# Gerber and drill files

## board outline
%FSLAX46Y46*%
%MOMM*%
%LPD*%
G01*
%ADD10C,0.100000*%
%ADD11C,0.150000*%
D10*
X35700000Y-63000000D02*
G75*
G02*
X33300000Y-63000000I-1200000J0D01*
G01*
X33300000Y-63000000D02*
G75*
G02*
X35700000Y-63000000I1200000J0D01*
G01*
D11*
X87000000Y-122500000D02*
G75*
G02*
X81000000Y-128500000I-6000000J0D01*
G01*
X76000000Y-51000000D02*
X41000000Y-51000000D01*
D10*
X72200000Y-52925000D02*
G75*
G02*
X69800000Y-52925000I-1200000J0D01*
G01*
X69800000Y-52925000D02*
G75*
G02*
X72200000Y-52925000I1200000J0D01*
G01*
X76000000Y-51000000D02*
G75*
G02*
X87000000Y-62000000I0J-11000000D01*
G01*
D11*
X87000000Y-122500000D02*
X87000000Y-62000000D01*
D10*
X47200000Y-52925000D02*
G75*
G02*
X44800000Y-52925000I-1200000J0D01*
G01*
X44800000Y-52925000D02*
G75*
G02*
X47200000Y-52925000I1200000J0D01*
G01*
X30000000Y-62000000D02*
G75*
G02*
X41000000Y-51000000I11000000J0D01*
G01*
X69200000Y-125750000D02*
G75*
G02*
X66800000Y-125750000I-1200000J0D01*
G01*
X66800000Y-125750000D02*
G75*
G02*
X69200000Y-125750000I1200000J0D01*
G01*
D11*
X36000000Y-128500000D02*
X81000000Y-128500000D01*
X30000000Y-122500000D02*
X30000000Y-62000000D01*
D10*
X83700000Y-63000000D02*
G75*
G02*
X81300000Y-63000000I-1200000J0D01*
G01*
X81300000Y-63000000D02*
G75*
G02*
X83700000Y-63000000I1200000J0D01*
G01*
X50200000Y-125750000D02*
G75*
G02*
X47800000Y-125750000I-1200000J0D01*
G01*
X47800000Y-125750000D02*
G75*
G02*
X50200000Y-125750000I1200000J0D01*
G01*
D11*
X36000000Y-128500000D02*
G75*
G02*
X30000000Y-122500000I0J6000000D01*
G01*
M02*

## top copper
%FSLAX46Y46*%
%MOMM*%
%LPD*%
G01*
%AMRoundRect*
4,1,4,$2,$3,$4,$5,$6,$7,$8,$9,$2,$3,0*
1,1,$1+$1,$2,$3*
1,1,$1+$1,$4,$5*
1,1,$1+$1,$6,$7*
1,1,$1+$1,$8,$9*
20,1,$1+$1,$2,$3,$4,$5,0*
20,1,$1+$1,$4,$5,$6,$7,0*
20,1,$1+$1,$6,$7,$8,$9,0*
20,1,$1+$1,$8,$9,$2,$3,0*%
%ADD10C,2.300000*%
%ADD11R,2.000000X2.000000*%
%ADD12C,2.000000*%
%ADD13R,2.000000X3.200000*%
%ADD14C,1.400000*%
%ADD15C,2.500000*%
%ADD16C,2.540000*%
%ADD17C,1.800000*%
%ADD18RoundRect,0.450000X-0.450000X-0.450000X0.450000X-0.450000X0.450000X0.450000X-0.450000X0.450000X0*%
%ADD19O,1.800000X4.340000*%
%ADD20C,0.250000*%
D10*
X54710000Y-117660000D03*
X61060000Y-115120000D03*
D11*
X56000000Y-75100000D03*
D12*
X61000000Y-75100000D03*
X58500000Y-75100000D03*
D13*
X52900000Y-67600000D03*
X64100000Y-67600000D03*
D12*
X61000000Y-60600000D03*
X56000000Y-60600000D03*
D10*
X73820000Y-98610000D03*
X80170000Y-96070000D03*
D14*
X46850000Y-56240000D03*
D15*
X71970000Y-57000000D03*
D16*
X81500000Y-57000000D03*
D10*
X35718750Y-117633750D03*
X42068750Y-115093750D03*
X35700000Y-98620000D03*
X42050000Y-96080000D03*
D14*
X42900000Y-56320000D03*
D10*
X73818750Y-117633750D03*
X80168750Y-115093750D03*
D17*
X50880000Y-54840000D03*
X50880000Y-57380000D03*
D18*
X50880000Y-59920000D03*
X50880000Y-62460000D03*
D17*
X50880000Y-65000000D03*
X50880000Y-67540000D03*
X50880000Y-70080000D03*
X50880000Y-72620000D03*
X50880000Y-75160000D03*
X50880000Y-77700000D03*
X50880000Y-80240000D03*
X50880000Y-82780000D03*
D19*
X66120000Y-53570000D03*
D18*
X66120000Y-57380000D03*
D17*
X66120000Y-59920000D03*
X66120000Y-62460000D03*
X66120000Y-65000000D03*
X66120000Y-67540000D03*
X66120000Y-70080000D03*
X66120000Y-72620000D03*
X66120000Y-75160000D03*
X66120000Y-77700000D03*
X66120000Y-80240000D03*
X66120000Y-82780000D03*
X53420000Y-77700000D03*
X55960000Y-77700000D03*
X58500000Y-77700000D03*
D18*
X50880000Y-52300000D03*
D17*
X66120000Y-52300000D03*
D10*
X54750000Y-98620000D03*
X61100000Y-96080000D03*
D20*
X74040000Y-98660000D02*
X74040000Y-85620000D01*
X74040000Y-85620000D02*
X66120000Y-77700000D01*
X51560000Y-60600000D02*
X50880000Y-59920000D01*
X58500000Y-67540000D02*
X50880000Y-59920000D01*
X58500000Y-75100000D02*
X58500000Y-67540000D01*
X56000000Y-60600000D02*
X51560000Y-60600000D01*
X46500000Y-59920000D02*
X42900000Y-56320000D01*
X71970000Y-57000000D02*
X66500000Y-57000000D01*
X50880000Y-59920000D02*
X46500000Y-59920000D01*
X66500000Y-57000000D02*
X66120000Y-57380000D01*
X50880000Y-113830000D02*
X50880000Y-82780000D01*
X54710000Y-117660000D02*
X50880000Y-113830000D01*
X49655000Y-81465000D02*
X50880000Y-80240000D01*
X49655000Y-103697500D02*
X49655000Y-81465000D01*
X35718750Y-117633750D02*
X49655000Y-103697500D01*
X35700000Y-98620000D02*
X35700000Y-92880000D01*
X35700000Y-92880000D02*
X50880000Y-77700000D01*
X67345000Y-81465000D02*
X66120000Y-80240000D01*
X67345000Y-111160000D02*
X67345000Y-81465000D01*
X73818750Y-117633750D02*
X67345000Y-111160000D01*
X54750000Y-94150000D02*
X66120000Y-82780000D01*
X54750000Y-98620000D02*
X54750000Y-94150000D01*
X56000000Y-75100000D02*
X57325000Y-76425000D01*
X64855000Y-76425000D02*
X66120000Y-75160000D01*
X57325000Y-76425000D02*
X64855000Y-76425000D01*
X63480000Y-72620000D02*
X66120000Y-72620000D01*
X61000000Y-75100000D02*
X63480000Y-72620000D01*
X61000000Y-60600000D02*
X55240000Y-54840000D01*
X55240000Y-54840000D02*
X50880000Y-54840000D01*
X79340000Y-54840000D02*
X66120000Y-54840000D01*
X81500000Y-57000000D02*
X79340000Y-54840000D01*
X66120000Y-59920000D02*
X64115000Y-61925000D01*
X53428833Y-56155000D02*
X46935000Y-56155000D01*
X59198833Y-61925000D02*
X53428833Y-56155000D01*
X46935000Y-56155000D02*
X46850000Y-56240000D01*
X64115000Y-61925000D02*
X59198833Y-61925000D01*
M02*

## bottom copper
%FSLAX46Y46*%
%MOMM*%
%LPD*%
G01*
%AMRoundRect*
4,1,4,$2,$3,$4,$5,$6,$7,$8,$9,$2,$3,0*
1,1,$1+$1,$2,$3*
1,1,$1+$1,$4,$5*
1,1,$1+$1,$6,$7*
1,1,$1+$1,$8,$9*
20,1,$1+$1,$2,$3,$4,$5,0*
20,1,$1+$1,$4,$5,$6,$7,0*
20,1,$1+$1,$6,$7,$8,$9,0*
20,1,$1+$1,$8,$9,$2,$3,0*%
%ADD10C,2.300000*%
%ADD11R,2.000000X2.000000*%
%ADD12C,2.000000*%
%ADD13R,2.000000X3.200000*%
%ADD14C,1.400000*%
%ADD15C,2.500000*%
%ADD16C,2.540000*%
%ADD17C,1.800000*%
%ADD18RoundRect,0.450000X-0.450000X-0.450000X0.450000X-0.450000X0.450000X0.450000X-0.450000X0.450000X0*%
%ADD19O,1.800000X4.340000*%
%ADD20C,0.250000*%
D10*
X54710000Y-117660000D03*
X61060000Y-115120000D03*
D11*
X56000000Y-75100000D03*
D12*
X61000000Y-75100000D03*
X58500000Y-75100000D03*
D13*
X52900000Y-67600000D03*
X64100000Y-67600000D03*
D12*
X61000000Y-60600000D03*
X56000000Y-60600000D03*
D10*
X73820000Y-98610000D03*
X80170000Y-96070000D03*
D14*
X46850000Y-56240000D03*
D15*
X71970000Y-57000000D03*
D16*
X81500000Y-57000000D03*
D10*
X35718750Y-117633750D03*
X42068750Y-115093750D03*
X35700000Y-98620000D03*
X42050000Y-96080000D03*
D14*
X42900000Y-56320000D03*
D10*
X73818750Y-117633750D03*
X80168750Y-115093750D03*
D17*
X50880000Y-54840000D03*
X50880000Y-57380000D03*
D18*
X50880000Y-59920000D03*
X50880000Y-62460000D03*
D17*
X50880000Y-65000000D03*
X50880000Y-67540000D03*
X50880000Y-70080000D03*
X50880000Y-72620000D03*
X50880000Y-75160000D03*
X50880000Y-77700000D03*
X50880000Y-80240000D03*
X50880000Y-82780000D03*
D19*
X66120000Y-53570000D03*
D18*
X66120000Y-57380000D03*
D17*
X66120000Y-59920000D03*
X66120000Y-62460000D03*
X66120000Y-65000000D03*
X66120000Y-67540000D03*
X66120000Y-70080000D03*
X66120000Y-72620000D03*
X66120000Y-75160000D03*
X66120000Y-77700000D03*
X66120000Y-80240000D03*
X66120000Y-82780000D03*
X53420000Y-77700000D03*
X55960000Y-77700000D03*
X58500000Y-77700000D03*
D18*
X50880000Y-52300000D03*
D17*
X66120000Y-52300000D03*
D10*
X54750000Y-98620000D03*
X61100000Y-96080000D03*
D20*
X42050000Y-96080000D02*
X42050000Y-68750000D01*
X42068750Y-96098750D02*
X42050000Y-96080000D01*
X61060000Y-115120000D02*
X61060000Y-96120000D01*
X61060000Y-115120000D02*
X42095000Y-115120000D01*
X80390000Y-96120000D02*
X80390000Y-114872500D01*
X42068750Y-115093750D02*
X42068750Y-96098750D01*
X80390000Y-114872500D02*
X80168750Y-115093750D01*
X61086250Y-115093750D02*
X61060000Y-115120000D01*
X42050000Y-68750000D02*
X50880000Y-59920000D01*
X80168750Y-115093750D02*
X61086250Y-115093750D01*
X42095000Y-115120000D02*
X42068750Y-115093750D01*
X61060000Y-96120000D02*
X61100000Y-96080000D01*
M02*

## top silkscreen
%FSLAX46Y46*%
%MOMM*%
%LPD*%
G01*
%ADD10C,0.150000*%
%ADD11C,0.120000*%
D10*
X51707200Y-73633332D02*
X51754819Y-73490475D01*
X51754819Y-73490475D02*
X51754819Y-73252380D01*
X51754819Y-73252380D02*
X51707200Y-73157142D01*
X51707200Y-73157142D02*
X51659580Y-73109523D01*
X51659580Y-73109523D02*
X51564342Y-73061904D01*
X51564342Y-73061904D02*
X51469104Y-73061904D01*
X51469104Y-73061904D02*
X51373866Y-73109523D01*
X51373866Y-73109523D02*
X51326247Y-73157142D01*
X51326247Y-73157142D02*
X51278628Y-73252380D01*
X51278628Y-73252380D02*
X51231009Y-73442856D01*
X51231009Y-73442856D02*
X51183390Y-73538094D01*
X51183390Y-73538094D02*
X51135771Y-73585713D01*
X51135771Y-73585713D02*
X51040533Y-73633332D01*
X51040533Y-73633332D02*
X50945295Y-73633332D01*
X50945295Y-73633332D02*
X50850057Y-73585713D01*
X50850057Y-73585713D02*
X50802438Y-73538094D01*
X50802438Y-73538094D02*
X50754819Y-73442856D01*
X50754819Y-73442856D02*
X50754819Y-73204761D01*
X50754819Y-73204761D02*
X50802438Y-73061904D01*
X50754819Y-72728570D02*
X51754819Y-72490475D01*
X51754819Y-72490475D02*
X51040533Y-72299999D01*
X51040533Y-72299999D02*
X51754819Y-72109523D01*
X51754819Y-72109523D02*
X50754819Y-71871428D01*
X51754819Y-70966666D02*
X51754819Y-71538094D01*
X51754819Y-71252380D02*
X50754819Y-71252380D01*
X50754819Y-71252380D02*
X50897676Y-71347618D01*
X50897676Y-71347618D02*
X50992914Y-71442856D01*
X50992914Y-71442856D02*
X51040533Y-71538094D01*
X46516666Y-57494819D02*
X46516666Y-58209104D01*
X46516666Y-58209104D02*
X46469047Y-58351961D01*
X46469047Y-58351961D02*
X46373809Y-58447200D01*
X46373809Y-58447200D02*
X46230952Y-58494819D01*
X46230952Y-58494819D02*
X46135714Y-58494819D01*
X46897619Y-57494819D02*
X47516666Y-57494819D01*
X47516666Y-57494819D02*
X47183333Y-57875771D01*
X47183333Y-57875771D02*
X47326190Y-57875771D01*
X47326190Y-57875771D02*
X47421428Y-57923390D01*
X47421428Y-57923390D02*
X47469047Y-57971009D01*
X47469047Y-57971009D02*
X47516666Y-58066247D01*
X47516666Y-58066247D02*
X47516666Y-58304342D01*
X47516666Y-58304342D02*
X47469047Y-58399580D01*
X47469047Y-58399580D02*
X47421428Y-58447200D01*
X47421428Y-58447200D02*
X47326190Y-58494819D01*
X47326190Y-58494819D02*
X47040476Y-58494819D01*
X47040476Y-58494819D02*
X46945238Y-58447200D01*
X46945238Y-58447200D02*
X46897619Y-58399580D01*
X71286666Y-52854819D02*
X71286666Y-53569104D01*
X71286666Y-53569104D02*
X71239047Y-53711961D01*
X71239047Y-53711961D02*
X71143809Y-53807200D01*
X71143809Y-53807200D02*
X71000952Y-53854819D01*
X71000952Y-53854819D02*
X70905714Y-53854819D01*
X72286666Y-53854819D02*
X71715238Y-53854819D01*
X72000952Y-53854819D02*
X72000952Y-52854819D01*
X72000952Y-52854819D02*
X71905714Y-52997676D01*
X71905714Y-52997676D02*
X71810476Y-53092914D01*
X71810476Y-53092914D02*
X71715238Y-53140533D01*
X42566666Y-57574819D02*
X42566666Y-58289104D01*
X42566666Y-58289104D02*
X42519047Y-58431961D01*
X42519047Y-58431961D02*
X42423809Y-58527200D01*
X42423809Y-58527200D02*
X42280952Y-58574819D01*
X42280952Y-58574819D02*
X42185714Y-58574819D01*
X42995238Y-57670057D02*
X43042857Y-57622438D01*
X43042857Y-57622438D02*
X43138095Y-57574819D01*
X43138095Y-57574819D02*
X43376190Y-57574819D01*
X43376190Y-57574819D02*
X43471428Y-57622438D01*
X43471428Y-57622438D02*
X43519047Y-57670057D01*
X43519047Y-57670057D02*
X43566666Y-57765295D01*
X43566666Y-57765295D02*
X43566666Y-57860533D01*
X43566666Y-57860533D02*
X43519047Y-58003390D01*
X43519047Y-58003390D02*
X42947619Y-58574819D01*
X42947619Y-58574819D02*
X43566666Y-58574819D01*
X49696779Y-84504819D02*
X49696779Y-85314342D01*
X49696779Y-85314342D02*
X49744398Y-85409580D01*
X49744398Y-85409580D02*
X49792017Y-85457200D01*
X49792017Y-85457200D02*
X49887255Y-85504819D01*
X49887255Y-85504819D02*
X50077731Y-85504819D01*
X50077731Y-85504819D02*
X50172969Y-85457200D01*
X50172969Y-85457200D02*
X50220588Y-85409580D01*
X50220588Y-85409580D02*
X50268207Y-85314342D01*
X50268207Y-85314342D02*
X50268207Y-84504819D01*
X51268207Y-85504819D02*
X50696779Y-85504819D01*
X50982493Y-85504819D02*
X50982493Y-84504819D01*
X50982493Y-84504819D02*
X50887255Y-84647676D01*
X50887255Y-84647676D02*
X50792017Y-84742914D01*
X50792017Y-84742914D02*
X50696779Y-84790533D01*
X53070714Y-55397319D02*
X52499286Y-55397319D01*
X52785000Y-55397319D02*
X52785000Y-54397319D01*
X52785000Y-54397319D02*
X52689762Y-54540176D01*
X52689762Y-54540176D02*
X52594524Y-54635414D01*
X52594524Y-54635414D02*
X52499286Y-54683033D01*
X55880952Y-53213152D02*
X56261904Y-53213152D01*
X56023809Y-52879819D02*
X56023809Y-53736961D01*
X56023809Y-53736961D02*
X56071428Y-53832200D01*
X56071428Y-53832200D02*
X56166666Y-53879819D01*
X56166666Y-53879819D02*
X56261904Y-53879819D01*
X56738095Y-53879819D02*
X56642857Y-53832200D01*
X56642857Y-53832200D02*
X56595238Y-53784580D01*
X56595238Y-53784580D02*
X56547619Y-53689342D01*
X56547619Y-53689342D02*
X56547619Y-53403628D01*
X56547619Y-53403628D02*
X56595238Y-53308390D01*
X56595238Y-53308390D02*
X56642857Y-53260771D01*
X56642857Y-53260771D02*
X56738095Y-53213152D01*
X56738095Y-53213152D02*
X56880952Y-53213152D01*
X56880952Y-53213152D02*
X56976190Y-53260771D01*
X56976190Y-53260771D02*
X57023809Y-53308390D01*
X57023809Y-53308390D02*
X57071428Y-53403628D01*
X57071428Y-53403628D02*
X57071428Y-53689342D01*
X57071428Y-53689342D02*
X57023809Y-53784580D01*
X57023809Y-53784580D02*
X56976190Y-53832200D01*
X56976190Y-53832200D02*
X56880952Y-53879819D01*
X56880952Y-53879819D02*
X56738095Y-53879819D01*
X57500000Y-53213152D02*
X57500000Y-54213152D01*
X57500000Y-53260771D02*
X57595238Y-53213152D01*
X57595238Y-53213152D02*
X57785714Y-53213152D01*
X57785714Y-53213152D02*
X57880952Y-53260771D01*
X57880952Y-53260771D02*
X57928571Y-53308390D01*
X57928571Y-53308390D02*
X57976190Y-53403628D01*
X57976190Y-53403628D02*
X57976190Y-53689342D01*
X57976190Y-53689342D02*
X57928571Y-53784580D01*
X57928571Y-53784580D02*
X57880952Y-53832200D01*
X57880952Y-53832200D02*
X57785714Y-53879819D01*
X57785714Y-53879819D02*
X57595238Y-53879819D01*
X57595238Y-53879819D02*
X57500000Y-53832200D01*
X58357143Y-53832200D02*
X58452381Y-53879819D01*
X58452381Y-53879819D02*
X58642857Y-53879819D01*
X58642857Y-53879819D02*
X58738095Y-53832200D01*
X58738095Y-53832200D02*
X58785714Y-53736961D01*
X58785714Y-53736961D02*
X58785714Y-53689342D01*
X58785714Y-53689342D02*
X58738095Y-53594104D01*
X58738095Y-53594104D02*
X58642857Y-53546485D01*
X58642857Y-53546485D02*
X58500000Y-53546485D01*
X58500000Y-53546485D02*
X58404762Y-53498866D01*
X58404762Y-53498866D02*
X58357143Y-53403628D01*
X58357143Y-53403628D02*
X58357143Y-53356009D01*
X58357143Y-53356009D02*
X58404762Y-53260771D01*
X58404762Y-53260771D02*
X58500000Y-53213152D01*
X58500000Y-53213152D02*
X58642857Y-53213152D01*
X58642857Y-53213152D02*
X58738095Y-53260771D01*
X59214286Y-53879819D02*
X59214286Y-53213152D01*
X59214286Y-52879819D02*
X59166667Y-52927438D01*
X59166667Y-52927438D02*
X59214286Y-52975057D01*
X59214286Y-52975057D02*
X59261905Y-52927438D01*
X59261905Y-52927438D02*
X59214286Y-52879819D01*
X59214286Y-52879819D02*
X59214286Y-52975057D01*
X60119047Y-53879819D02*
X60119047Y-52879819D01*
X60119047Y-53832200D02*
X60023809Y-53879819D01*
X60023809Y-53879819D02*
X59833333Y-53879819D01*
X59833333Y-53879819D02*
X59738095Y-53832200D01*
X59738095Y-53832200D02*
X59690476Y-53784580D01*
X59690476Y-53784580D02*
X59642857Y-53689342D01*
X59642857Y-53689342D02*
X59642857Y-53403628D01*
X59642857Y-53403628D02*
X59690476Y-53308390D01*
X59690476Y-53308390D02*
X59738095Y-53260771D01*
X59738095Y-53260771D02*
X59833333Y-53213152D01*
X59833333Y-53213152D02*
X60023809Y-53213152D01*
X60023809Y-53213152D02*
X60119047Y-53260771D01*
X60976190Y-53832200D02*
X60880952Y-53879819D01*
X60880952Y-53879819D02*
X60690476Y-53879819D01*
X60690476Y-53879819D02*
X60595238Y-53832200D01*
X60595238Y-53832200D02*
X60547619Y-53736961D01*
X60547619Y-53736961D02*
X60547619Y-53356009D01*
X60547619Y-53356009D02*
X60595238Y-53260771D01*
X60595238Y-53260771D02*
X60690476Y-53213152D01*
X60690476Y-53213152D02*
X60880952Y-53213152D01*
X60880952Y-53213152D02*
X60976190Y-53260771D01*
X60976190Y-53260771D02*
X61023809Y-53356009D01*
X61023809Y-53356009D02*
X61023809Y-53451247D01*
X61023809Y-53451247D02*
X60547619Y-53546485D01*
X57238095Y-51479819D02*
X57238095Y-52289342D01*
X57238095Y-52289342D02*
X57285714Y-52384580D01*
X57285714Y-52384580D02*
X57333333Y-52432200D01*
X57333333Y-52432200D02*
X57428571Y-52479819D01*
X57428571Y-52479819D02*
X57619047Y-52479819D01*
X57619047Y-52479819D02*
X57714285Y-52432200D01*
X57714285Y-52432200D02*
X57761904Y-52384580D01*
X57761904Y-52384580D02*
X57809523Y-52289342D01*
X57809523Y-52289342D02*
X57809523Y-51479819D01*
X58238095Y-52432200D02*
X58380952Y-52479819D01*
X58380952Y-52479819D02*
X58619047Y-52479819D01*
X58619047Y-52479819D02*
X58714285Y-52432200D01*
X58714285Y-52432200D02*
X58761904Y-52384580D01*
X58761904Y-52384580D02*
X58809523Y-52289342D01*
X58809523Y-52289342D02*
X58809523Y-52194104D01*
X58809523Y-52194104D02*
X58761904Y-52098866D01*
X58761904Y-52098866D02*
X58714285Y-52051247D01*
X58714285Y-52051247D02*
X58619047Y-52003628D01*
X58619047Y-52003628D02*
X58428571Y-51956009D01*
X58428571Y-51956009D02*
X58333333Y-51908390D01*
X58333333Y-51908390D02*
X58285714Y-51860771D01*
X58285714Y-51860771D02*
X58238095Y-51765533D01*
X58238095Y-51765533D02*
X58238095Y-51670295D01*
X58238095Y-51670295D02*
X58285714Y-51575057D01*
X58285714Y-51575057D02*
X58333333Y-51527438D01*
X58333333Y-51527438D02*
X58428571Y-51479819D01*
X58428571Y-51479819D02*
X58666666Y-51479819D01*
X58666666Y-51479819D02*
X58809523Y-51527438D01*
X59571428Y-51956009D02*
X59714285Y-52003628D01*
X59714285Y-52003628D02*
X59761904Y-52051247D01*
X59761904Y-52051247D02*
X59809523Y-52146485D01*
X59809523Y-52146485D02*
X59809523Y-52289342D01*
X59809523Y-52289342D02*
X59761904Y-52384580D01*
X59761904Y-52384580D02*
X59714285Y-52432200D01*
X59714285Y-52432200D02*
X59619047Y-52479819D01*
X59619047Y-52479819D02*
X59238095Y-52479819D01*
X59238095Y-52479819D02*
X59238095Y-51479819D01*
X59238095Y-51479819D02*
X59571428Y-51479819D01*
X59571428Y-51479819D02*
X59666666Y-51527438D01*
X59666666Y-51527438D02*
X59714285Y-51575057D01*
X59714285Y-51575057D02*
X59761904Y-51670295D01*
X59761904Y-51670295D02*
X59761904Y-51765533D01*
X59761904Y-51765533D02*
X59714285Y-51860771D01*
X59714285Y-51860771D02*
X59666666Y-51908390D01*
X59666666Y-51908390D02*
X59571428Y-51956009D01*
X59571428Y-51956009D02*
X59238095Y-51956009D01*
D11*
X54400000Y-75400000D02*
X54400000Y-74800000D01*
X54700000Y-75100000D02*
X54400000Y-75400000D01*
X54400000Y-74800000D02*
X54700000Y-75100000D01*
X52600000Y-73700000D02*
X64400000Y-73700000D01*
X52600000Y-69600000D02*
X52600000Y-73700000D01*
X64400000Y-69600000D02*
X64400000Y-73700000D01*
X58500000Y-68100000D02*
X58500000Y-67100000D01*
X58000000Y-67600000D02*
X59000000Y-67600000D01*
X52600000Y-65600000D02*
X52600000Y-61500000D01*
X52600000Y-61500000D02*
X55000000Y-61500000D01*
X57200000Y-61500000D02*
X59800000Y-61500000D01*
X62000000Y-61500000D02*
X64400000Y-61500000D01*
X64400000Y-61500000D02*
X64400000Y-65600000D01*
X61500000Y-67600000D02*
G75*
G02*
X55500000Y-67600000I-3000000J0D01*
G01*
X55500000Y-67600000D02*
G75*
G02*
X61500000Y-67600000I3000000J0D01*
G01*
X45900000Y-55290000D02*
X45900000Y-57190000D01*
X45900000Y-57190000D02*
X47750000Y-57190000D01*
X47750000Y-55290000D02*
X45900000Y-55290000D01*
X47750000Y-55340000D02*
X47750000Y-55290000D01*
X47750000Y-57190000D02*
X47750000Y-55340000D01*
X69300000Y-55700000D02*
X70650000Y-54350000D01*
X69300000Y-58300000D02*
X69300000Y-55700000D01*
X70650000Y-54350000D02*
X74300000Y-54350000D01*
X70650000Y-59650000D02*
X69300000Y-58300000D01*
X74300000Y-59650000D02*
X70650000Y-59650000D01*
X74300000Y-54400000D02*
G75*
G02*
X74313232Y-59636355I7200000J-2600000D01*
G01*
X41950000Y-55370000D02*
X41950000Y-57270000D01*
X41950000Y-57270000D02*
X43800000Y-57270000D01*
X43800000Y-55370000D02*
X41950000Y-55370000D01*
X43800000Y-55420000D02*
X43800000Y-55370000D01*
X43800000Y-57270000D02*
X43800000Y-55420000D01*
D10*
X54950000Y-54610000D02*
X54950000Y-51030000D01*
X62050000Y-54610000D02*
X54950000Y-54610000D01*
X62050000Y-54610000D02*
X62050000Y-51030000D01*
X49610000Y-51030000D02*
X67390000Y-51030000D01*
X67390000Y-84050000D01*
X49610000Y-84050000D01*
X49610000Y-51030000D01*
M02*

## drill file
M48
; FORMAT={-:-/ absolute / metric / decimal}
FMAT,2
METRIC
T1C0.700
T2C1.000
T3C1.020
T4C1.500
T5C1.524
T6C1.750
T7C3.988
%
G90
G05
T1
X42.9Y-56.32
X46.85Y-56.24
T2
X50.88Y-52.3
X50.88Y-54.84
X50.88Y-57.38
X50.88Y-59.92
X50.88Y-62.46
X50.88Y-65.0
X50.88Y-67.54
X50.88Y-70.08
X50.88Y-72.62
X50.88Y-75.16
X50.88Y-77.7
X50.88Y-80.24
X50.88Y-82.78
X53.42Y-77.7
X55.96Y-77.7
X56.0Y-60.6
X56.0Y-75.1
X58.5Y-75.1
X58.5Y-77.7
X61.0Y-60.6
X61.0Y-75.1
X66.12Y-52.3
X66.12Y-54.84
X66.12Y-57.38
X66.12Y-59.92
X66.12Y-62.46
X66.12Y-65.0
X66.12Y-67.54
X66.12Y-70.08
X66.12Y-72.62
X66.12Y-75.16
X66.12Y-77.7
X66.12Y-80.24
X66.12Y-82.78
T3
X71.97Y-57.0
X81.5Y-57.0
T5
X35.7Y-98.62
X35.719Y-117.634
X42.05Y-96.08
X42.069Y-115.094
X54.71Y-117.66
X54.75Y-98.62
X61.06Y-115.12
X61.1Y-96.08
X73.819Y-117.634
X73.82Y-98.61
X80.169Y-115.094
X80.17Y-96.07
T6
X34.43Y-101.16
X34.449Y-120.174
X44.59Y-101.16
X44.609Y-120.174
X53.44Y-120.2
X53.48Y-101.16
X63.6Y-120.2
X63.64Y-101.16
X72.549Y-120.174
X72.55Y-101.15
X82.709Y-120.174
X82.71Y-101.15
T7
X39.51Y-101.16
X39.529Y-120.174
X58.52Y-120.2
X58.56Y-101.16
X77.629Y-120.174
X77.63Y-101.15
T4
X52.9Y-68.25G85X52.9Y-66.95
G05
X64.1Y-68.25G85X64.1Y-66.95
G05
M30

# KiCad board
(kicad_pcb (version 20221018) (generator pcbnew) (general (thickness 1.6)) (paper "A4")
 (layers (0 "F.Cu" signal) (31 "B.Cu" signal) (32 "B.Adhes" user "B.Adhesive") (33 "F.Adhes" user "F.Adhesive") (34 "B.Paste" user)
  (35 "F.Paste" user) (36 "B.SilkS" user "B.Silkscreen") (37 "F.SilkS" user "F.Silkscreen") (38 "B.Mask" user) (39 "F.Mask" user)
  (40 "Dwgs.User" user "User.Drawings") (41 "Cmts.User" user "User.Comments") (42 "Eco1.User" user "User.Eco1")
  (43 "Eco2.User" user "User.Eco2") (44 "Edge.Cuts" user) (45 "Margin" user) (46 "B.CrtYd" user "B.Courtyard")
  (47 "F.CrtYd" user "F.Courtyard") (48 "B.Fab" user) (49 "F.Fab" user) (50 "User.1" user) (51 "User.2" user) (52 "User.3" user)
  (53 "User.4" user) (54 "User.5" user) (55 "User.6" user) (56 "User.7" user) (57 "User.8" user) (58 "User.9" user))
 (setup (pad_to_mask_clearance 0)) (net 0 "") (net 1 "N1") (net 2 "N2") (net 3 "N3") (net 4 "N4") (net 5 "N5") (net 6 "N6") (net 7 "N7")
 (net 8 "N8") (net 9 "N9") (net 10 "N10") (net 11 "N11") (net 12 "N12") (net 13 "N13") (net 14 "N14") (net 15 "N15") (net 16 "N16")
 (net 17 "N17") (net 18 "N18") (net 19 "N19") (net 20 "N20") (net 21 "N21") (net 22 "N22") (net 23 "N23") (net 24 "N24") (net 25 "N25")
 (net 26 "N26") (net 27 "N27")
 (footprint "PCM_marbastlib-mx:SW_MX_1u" (layer "F.Cu") (at 58.52 120.2)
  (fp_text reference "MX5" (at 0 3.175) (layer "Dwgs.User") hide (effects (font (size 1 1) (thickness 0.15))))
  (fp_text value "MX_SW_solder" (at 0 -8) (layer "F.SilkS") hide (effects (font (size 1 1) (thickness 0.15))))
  (pad "" np_thru_hole circle (at -5.08 0) (size 1.75 1.75) (drill 1.75) (layers "*.Cu" "*.Mask"))
  (pad "" np_thru_hole circle (at 0 0) (size 3.9878 3.9878) (drill 3.9878) (layers "*.Cu" "*.Mask"))
  (pad "" np_thru_hole circle (at 5.08 0) (size 1.75 1.75) (drill 1.75) (layers "*.Cu" "*.Mask"))
  (pad "1" thru_hole circle (at -3.81 -2.54) (size 2.3 2.3) (drill 1.524) (layers "*.Cu" "B.Mask") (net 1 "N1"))
  (pad "2" thru_hole circle (at 2.54 -5.08) (size 2.3 2.3) (drill 1.524) (layers "*.Cu" "B.Mask") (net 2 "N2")))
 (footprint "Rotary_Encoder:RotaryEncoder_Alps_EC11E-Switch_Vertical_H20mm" (layer "F.Cu") (at 56 75.1 90)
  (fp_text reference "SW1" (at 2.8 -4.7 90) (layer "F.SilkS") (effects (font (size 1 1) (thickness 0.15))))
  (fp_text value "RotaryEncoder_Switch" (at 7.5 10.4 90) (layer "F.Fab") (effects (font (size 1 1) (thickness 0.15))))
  (fp_line (start -0.3 -1.6) (end 0.3 -1.6) (stroke (width 0.12) (type solid)) (layer "F.SilkS"))
  (fp_line (start 0 -1.3) (end -0.3 -1.6) (stroke (width 0.12) (type solid)) (layer "F.SilkS"))
  (fp_line (start 0.3 -1.6) (end 0 -1.3) (stroke (width 0.12) (type solid)) (layer "F.SilkS"))
  (fp_line (start 1.4 -3.4) (end 1.4 8.4) (stroke (width 0.12) (type solid)) (layer "F.SilkS"))
  (fp_line (start 5.5 -3.4) (end 1.4 -3.4) (stroke (width 0.12) (type solid)) (layer "F.SilkS"))
  (fp_line (start 5.5 8.4) (end 1.4 8.4) (stroke (width 0.12) (type solid)) (layer "F.SilkS"))
  (fp_line (start 7 2.5) (end 8 2.5) (stroke (width 0.12) (type solid)) (layer "F.SilkS"))
  (fp_line (start 7.5 2) (end 7.5 3) (stroke (width 0.12) (type solid)) (layer "F.SilkS"))
  (fp_line (start 9.5 -3.4) (end 13.6 -3.4) (stroke (width 0.12) (type solid)) (layer "F.SilkS"))
  (fp_line (start 13.6 -3.4) (end 13.6 -1) (stroke (width 0.12) (type solid)) (layer "F.SilkS"))
  (fp_line (start 13.6 1.2) (end 13.6 3.8) (stroke (width 0.12) (type solid)) (layer "F.SilkS"))
  (fp_line (start 13.6 6) (end 13.6 8.4) (stroke (width 0.12) (type solid)) (layer "F.SilkS"))
  (fp_line (start 13.6 8.4) (end 9.5 8.4) (stroke (width 0.12) (type solid)) (layer "F.SilkS"))
  (fp_circle (center 7.5 2.5) (end 10.5 2.5) (stroke (width 0.12) (type solid)) (fill none) (layer "F.SilkS"))
  (pad "A" thru_hole rect (at 0 0 90) (size 2 2) (drill 1) (layers "*.Cu" "*.Mask") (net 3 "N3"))
  (pad "B" thru_hole circle (at 0 5 90) (size 2 2) (drill 1) (layers "*.Cu" "*.Mask") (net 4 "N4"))
  (pad "C" thru_hole circle (at 0 2.5 90) (size 2 2) (drill 1) (layers "*.Cu" "*.Mask") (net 2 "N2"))
  (pad "MP" thru_hole rect (at 7.5 -3.1 90) (size 3.2 2) (drill oval 2.8 1.5) (layers "*.Cu" "*.Mask"))
  (pad "MP" thru_hole rect (at 7.5 8.1 90) (size 3.2 2) (drill oval 2.8 1.5) (layers "*.Cu" "*.Mask"))
  (pad "S1" thru_hole circle (at 14.5 5 90) (size 2 2) (drill 1) (layers "*.Cu" "*.Mask") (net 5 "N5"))
  (pad "S2" thru_hole circle (at 14.5 0 90) (size 2 2) (drill 1) (layers "*.Cu" "*.Mask") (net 2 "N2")))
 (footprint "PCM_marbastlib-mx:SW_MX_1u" (layer "F.Cu") (at 77.63 101.15)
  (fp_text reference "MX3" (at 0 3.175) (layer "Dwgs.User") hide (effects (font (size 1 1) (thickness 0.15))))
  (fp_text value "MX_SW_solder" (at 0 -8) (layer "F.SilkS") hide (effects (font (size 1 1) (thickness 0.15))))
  (pad "" np_thru_hole circle (at -5.08 0) (size 1.75 1.75) (drill 1.75) (layers "*.Cu" "*.Mask"))
  (pad "" np_thru_hole circle (at 0 0) (size 3.9878 3.9878) (drill 3.9878) (layers "*.Cu" "*.Mask"))
  (pad "" np_thru_hole circle (at 5.08 0) (size 1.75 1.75) (drill 1.75) (layers "*.Cu" "*.Mask"))
  (pad "1" thru_hole circle (at -3.81 -2.54) (size 2.3 2.3) (drill 1.524) (layers "*.Cu" "B.Mask") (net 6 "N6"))
  (pad "2" thru_hole circle (at 2.54 -5.08) (size 2.3 2.3) (drill 1.524) (layers "*.Cu" "B.Mask") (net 2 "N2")))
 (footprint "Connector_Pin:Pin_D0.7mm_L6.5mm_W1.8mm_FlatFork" (layer "F.Cu") (at 46.85 56.24)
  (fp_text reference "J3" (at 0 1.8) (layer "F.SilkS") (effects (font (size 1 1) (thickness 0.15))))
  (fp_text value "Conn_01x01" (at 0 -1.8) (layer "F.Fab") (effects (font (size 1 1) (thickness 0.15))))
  (fp_line (start -0.95 -0.95) (end -0.95 0.95) (stroke (width 0.12) (type solid)) (layer "F.SilkS"))
  (fp_line (start -0.95 0.95) (end 0.9 0.95) (stroke (width 0.12) (type solid)) (layer "F.SilkS"))
  (fp_line (start 0.9 -0.95) (end -0.95 -0.95) (stroke (width 0.12) (type solid)) (layer "F.SilkS"))
  (fp_line (start 0.9 -0.9) (end 0.9 -0.95) (stroke (width 0.12) (type solid)) (layer "F.SilkS"))
  (fp_line (start 0.9 0.95) (end 0.9 -0.9) (stroke (width 0.12) (type solid)) (layer "F.SilkS"))
  (pad "1" thru_hole circle (at 0 0) (size 1.4 1.4) (drill 0.7) (layers "*.Cu" "*.Mask") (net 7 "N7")))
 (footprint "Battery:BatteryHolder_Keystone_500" (layer "F.Cu") (at 71.97 57)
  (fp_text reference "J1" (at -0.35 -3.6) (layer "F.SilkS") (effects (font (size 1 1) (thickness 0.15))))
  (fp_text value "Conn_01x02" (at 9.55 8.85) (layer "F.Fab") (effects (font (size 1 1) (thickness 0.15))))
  (fp_line (start -2.67 -1.3) (end -1.32 -2.65) (stroke (width 0.12) (type solid)) (layer "F.SilkS"))
  (fp_line (start -2.67 1.3) (end -2.67 -1.3) (stroke (width 0.12) (type solid)) (layer "F.SilkS"))
  (fp_line (start -1.32 -2.65) (end 2.33 -2.65) (stroke (width 0.12) (type solid)) (layer "F.SilkS"))
  (fp_line (start -1.32 2.65) (end -2.67 1.3) (stroke (width 0.12) (type solid)) (layer "F.SilkS"))
  (fp_line (start 2.33 2.65) (end -1.32 2.65) (stroke (width 0.12) (type solid)) (layer "F.SilkS"))
  (fp_arc (start 2.33 -2.6) (mid 17.185039 -0.019344) (end 2.343232 2.636355) (stroke (width 0.12) (type solid)) (layer "F.SilkS"))
  (pad "1" thru_hole circle (at 0 0) (size 2.5 2.5) (drill 1.02) (layers "*.Cu" "*.Mask") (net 2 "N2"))
  (pad "2" thru_hole circle (at 9.53 0) (size 2.54 2.54) (drill 1.02) (layers "*.Cu" "*.Mask") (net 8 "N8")))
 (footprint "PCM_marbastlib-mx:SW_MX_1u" (layer "F.Cu") (at 39.52875 120.17375)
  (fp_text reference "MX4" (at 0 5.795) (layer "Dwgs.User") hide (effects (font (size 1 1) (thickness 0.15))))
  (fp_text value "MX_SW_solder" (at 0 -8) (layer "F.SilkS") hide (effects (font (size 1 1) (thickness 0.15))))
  (pad "" np_thru_hole circle (at -5.08 0) (size 1.75 1.75) (drill 1.75) (layers "*.Cu" "*.Mask"))
  (pad "" np_thru_hole circle (at 0 0) (size 3.9878 3.9878) (drill 3.9878) (layers "*.Cu" "*.Mask"))
  (pad "" np_thru_hole circle (at 5.08 0) (size 1.75 1.75) (drill 1.75) (layers "*.Cu" "*.Mask"))
  (pad "1" thru_hole circle (at -3.81 -2.54) (size 2.3 2.3) (drill 1.524) (layers "*.Cu" "B.Mask") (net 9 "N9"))
  (pad "2" thru_hole circle (at 2.54 -5.08) (size 2.3 2.3) (drill 1.524) (layers "*.Cu" "B.Mask") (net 2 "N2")))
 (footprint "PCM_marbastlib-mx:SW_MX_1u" (layer "F.Cu") (at 39.51 101.16)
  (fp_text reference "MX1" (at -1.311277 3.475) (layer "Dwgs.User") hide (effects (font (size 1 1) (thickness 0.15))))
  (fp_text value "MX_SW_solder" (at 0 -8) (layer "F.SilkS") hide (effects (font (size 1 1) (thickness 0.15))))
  (pad "" np_thru_hole circle (at -5.08 0) (size 1.75 1.75) (drill 1.75) (layers "*.Cu" "*.Mask"))
  (pad "" np_thru_hole circle (at 0 0) (size 3.9878 3.9878) (drill 3.9878) (layers "*.Cu" "*.Mask"))
  (pad "" np_thru_hole circle (at 5.08 0) (size 1.75 1.75) (drill 1.75) (layers "*.Cu" "*.Mask"))
  (pad "1" thru_hole circle (at -3.81 -2.54) (size 2.3 2.3) (drill 1.524) (layers "*.Cu" "B.Mask") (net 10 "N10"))
  (pad "2" thru_hole circle (at 2.54 -5.08) (size 2.3 2.3) (drill 1.524) (layers "*.Cu" "B.Mask") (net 2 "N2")))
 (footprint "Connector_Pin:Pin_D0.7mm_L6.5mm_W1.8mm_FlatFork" (layer "F.Cu") (at 42.9 56.32)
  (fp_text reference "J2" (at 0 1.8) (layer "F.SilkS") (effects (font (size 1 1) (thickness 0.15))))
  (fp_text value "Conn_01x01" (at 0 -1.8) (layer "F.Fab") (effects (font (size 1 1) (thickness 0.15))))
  (fp_line (start -0.95 -0.95) (end -0.95 0.95) (stroke (width 0.12) (type solid)) (layer "F.SilkS"))
  (fp_line (start -0.95 0.95) (end 0.9 0.95) (stroke (width 0.12) (type solid)) (layer "F.SilkS"))
  (fp_line (start 0.9 -0.95) (end -0.95 -0.95) (stroke (width 0.12) (type solid)) (layer "F.SilkS"))
  (fp_line (start 0.9 -0.9) (end 0.9 -0.95) (stroke (width 0.12) (type solid)) (layer "F.SilkS"))
  (fp_line (start 0.9 0.95) (end 0.9 -0.9) (stroke (width 0.12) (type solid)) (layer "F.SilkS"))
  (pad "1" thru_hole circle (at 0 0) (size 1.4 1.4) (drill 0.7) (layers "*.Cu" "*.Mask") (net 2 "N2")))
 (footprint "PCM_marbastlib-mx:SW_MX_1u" (layer "F.Cu") (at 77.62875 120.17375)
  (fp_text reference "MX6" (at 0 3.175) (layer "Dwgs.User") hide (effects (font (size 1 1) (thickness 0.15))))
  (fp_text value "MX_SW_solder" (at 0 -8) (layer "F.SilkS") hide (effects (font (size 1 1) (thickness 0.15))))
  (pad "" np_thru_hole circle (at -5.08 0) (size 1.75 1.75) (drill 1.75) (layers "*.Cu" "*.Mask"))
  (pad "" np_thru_hole circle (at 0 0) (size 3.9878 3.9878) (drill 3.9878) (layers "*.Cu" "*.Mask"))
  (pad "" np_thru_hole circle (at 5.08 0) (size 1.75 1.75) (drill 1.75) (layers "*.Cu" "*.Mask"))
  (pad "1" thru_hole circle (at -3.81 -2.54) (size 2.3 2.3) (drill 1.524) (layers "*.Cu" "B.Mask") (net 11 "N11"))
  (pad "2" thru_hole circle (at 2.54 -5.08) (size 2.3 2.3) (drill 1.524) (layers "*.Cu" "B.Mask") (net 2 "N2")))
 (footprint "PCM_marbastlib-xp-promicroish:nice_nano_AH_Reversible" (layer "F.Cu") (at 58.5 68.81)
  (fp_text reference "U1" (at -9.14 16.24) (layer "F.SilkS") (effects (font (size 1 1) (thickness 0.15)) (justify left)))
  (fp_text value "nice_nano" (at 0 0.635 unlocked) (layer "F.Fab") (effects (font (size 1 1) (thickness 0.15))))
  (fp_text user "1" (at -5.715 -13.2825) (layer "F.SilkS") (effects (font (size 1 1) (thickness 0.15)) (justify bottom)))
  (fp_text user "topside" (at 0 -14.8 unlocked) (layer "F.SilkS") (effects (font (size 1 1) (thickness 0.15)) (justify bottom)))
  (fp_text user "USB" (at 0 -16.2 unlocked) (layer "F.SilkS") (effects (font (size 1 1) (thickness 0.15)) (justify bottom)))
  (fp_line (start -3.55 -14.2) (end -3.55 -17.78) (stroke (width 0.15) (type default)) (layer "F.SilkS"))
  (fp_line (start 3.55 -14.2) (end -3.55 -14.2) (stroke (width 0.15) (type default)) (layer "F.SilkS"))
  (fp_line (start 3.55 -14.2) (end 3.55 -17.78) (stroke (width 0.15) (type default)) (layer "F.SilkS"))
  (fp_rect (start -8.89 -17.78) (end 8.89 15.24) (stroke (width 0.15) (type solid)) (fill none) (layer "F.SilkS"))
  (pad "1" thru_hole circle (at -7.62 -13.97) (size 1.8 1.8) (drill 1) (layers "*.Cu" "*.Mask") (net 5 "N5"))
  (pad "2" thru_hole circle (at -7.62 -11.43) (size 1.8 1.8) (drill 1) (layers "*.Cu" "*.Mask") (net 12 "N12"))
  (pad "3" thru_hole roundrect (at -7.62 -8.89) (size 1.8 1.8) (drill 1) (layers "*.Cu" "*.Mask") (roundrect_rratio 0.25) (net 2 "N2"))
  (pad "4" thru_hole roundrect (at -7.62 -6.35) (size 1.8 1.8) (drill 1) (layers "*.Cu" "*.Mask") (roundrect_rratio 0.25) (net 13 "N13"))
  (pad "5" thru_hole circle (at -7.62 -3.81) (size 1.8 1.8) (drill 1) (layers "*.Cu" "*.Mask") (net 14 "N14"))
  (pad "6" thru_hole circle (at -7.62 -1.27) (size 1.8 1.8) (drill 1) (layers "*.Cu" "*.Mask") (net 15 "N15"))
  (pad "7" thru_hole circle (at -7.62 1.27) (size 1.8 1.8) (drill 1) (layers "*.Cu" "*.Mask") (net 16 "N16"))
  (pad "8" thru_hole circle (at -7.62 3.81) (size 1.8 1.8) (drill 1) (layers "*.Cu" "*.Mask") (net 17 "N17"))
  (pad "9" thru_hole circle (at -7.62 6.35) (size 1.8 1.8) (drill 1) (layers "*.Cu" "*.Mask") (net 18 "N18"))
  (pad "10" thru_hole circle (at -7.62 8.89) (size 1.8 1.8) (drill 1) (layers "*.Cu" "*.Mask") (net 10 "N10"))
  (pad "11" thru_hole circle (at -7.62 11.43) (size 1.8 1.8) (drill 1) (layers "*.Cu" "*.Mask") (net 9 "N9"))
  (pad "12" thru_hole circle (at -7.62 13.97) (size 1.8 1.8) (drill 1) (layers "*.Cu" "*.Mask") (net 1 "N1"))
  (pad "13" thru_hole oval (at 7.62 -13.97) (size 1.8 4.34) (drill 1 (offset 0 -1.27)) (layers "*.Cu" "*.Mask") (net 8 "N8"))
  (pad "14" thru_hole roundrect (at 7.62 -11.43) (size 1.8 1.8) (drill 1) (layers "*.Cu" "*.Mask") (roundrect_rratio 0.25) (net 2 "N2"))
  (pad "15" thru_hole circle (at 7.62 -8.89) (size 1.8 1.8) (drill 1) (layers "*.Cu" "*.Mask") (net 7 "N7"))
  (pad "16" thru_hole circle (at 7.62 -6.35) (size 1.8 1.8) (drill 1) (layers "*.Cu" "*.Mask") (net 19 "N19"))
  (pad "17" thru_hole circle (at 7.62 -3.81) (size 1.8 1.8) (drill 1) (layers "*.Cu" "*.Mask") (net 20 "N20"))
  (pad "18" thru_hole circle (at 7.62 -1.27) (size 1.8 1.8) (drill 1) (layers "*.Cu" "*.Mask") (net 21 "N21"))
  (pad "19" thru_hole circle (at 7.62 1.27) (size 1.8 1.8) (drill 1) (layers "*.Cu" "*.Mask") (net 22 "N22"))
  (pad "20" thru_hole circle (at 7.62 3.81) (size 1.8 1.8) (drill 1) (layers "*.Cu" "*.Mask") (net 4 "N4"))
  (pad "21" thru_hole circle (at 7.62 6.35) (size 1.8 1.8) (drill 1) (layers "*.Cu" "*.Mask") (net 3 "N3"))
  (pad "22" thru_hole circle (at 7.62 8.89) (size 1.8 1.8) (drill 1) (layers "*.Cu" "*.Mask") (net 6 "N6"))
  (pad "23" thru_hole circle (at 7.62 11.43) (size 1.8 1.8) (drill 1) (layers "*.Cu" "*.Mask") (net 11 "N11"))
  (pad "24" thru_hole circle (at 7.62 13.97) (size 1.8 1.8) (drill 1) (layers "*.Cu" "*.Mask") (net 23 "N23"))
  (pad "25" thru_hole circle (at -5.08 8.89) (size 1.8 1.8) (drill 1) (layers "*.Cu" "*.Mask") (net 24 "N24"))
  (pad "26" thru_hole circle (at -2.54 8.89) (size 1.8 1.8) (drill 1) (layers "*.Cu" "*.Mask") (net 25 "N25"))
  (pad "27" thru_hole circle (at 0 8.89) (size 1.8 1.8) (drill 1) (layers "*.Cu" "*.Mask") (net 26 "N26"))
  (pad "28" thru_hole roundrect (at -7.62 -16.51) (size 1.8 1.8) (drill 1) (layers "*.Cu" "*.Mask") (roundrect_rratio 0.25) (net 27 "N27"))
  (pad "29" thru_hole circle (at 7.62 -16.51) (size 1.8 1.8) (drill 1) (layers "*.Cu" "*.Mask") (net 8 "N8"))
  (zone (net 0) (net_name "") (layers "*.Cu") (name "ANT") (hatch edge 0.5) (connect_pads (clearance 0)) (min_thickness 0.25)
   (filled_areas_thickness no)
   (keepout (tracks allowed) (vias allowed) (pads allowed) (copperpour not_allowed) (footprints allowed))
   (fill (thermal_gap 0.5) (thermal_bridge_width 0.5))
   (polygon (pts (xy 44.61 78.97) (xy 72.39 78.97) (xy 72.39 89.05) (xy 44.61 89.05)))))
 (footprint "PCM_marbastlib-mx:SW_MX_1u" (layer "F.Cu") (at 58.56 101.16)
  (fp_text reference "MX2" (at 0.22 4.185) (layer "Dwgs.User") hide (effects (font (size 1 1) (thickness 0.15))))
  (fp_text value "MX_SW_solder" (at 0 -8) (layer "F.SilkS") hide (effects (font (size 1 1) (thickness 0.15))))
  (pad "" np_thru_hole circle (at -5.08 0) (size 1.75 1.75) (drill 1.75) (layers "*.Cu" "*.Mask"))
  (pad "" np_thru_hole circle (at 0 0) (size 3.9878 3.9878) (drill 3.9878) (layers "*.Cu" "*.Mask"))
  (pad "" np_thru_hole circle (at 5.08 0) (size 1.75 1.75) (drill 1.75) (layers "*.Cu" "*.Mask"))
  (pad "1" thru_hole circle (at -3.81 -2.54) (size 2.3 2.3) (drill 1.524) (layers "*.Cu" "B.Mask") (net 23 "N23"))
  (pad "2" thru_hole circle (at 2.54 -5.08) (size 2.3 2.3) (drill 1.524) (layers "*.Cu" "B.Mask") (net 2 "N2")))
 (gr_circle (center 34.5 63) (end 35.7 63) (stroke (width 0.1) (type default)) (fill none) (layer "Edge.Cuts"))
 (gr_arc (start 87 122.5) (mid 85.242641 126.742641) (end 81 128.5) (stroke (width 0.15) (type default)) (layer "Edge.Cuts"))
 (gr_line (start 76 51) (end 41 51) (stroke (width 0.15) (type default)) (layer "Edge.Cuts"))
 (gr_circle (center 71 52.925) (end 72.2 52.925) (stroke (width 0.1) (type default)) (fill none) (layer "Edge.Cuts"))
 (gr_arc (start 76 51) (mid 83.778175 54.221825) (end 87 62) (stroke (width 0.1) (type default)) (layer "Edge.Cuts"))
 (gr_line (start 87 122.5) (end 87 62) (stroke (width 0.15) (type default)) (layer "Edge.Cuts"))
 (gr_circle (center 46 52.925) (end 47.2 52.925) (stroke (width 0.1) (type default)) (fill none) (layer "Edge.Cuts"))
 (gr_arc (start 30 62) (mid 33.221825 54.221825) (end 41 51) (stroke (width 0.1) (type default)) (layer "Edge.Cuts"))
 (gr_circle (center 68 125.75) (end 69.2 125.75) (stroke (width 0.1) (type default)) (fill none) (layer "Edge.Cuts"))
 (gr_line (start 36 128.5) (end 81 128.5) (stroke (width 0.15) (type default)) (layer "Edge.Cuts"))
 (gr_line (start 30 122.5) (end 30 62) (stroke (width 0.15) (type default)) (layer "Edge.Cuts"))
 (gr_circle (center 82.5 63) (end 83.7 63) (stroke (width 0.1) (type default)) (fill none) (layer "Edge.Cuts"))
 (gr_circle (center 49 125.75) (end 50.2 125.75) (stroke (width 0.1) (type default)) (fill none) (layer "Edge.Cuts"))
 (gr_arc (start 36 128.5) (mid 31.757359 126.742641) (end 30 122.5) (stroke (width 0.15) (type default)) (layer "Edge.Cuts"))
 (segment (start 74.04 98.66) (end 74.04 85.62) (width 0.25) (layer "F.Cu") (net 6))
 (segment (start 74.04 85.62) (end 66.12 77.7) (width 0.25) (layer "F.Cu") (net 6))
 (segment (start 51.56 60.6) (end 50.88 59.92) (width 0.25) (layer "F.Cu") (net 2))
 (segment (start 58.5 67.54) (end 50.88 59.92) (width 0.25) (layer "F.Cu") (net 2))
 (segment (start 58.5 75.1) (end 58.5 67.54) (width 0.25) (layer "F.Cu") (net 2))
 (segment (start 56 60.6) (end 51.56 60.6) (width 0.25) (layer "F.Cu") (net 2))
 (segment (start 46.5 59.92) (end 42.9 56.32) (width 0.25) (layer "F.Cu") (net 2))
 (segment (start 71.97 57) (end 66.5 57) (width 0.25) (layer "F.Cu") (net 2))
 (segment (start 50.88 59.92) (end 46.5 59.92) (width 0.25) (layer "F.Cu") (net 2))
 (segment (start 66.5 57) (end 66.12 57.38) (width 0.25) (layer "F.Cu") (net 2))
 (segment (start 42.05 96.08) (end 42.05 68.75) (width 0.25) (layer "B.Cu") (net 2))
 (segment (start 42.06875 96.09875) (end 42.05 96.08) (width 0.25) (layer "B.Cu") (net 2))
 (segment (start 61.06 115.12) (end 61.06 96.12) (width 0.25) (layer "B.Cu") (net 2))
 (segment (start 61.06 115.12) (end 42.095 115.12) (width 0.25) (layer "B.Cu") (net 2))
 (segment (start 80.39 96.12) (end 80.39 114.8725) (width 0.25) (layer "B.Cu") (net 2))
 (segment (start 42.06875 115.09375) (end 42.06875 96.09875) (width 0.25) (layer "B.Cu") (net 2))
 (segment (start 80.39 114.8725) (end 80.16875 115.09375) (width 0.25) (layer "B.Cu") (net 2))
 (segment (start 61.08625 115.09375) (end 61.06 115.12) (width 0.25) (layer "B.Cu") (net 2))
 (segment (start 42.05 68.75) (end 50.88 59.92) (width 0.25) (layer "B.Cu") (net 2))
 (segment (start 80.16875 115.09375) (end 61.08625 115.09375) (width 0.25) (layer "B.Cu") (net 2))
 (segment (start 42.095 115.12) (end 42.06875 115.09375) (width 0.25) (layer "B.Cu") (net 2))
 (segment (start 61.06 96.12) (end 61.1 96.08) (width 0.25) (layer "B.Cu") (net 2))
 (segment (start 50.88 113.83) (end 50.88 82.78) (width 0.25) (layer "F.Cu") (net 1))
 (segment (start 54.71 117.66) (end 50.88 113.83) (width 0.25) (layer "F.Cu") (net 1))
 (segment (start 49.655 81.465) (end 50.88 80.24) (width 0.25) (layer "F.Cu") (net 9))
 (segment (start 49.655 103.6975) (end 49.655 81.465) (width 0.25) (layer "F.Cu") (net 9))
 (segment (start 35.71875 117.63375) (end 49.655 103.6975) (width 0.25) (layer "F.Cu") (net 9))
 (segment (start 35.7 98.62) (end 35.7 92.88) (width 0.25) (layer "F.Cu") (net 10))
 (segment (start 35.7 92.88) (end 50.88 77.7) (width 0.25) (layer "F.Cu") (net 10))
 (segment (start 67.345 81.465) (end 66.12 80.24) (width 0.25) (layer "F.Cu") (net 11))
 (segment (start 67.345 111.16) (end 67.345 81.465) (width 0.25) (layer "F.Cu") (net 11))
 (segment (start 73.81875 117.63375) (end 67.345 111.16) (width 0.25) (layer "F.Cu") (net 11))
 (segment (start 54.75 94.15) (end 66.12 82.78) (width 0.25) (layer "F.Cu") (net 23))
 (segment (start 54.75 98.62) (end 54.75 94.15) (width 0.25) (layer "F.Cu") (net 23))
 (segment (start 56 75.1) (end 57.325 76.425) (width 0.25) (layer "F.Cu") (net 3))
 (segment (start 64.855 76.425) (end 66.12 75.16) (width 0.25) (layer "F.Cu") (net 3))
 (segment (start 57.325 76.425) (end 64.855 76.425) (width 0.25) (layer "F.Cu") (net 3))
 (segment (start 63.48 72.62) (end 66.12 72.62) (width 0.25) (layer "F.Cu") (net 4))
 (segment (start 61 75.1) (end 63.48 72.62) (width 0.25) (layer "F.Cu") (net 4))
 (segment (start 61 60.6) (end 55.24 54.84) (width 0.25) (layer "F.Cu") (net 5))
 (segment (start 55.24 54.84) (end 50.88 54.84) (width 0.25) (layer "F.Cu") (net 5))
 (segment (start 79.34 54.84) (end 66.12 54.84) (width 0.25) (layer "F.Cu") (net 8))
 (segment (start 81.5 57) (end 79.34 54.84) (width 0.25) (layer "F.Cu") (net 8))
 (segment (start 66.12 59.92) (end 64.115 61.925) (width 0.25) (layer "F.Cu") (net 7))
 (segment (start 53.428833 56.155) (end 46.935 56.155) (width 0.25) (layer "F.Cu") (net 7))
 (segment (start 59.198833 61.925) (end 53.428833 56.155) (width 0.25) (layer "F.Cu") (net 7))
 (segment (start 46.935 56.155) (end 46.85 56.24) (width 0.25) (layer "F.Cu") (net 7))
 (segment (start 64.115 61.925) (end 59.198833 61.925) (width 0.25) (layer "F.Cu") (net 7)))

